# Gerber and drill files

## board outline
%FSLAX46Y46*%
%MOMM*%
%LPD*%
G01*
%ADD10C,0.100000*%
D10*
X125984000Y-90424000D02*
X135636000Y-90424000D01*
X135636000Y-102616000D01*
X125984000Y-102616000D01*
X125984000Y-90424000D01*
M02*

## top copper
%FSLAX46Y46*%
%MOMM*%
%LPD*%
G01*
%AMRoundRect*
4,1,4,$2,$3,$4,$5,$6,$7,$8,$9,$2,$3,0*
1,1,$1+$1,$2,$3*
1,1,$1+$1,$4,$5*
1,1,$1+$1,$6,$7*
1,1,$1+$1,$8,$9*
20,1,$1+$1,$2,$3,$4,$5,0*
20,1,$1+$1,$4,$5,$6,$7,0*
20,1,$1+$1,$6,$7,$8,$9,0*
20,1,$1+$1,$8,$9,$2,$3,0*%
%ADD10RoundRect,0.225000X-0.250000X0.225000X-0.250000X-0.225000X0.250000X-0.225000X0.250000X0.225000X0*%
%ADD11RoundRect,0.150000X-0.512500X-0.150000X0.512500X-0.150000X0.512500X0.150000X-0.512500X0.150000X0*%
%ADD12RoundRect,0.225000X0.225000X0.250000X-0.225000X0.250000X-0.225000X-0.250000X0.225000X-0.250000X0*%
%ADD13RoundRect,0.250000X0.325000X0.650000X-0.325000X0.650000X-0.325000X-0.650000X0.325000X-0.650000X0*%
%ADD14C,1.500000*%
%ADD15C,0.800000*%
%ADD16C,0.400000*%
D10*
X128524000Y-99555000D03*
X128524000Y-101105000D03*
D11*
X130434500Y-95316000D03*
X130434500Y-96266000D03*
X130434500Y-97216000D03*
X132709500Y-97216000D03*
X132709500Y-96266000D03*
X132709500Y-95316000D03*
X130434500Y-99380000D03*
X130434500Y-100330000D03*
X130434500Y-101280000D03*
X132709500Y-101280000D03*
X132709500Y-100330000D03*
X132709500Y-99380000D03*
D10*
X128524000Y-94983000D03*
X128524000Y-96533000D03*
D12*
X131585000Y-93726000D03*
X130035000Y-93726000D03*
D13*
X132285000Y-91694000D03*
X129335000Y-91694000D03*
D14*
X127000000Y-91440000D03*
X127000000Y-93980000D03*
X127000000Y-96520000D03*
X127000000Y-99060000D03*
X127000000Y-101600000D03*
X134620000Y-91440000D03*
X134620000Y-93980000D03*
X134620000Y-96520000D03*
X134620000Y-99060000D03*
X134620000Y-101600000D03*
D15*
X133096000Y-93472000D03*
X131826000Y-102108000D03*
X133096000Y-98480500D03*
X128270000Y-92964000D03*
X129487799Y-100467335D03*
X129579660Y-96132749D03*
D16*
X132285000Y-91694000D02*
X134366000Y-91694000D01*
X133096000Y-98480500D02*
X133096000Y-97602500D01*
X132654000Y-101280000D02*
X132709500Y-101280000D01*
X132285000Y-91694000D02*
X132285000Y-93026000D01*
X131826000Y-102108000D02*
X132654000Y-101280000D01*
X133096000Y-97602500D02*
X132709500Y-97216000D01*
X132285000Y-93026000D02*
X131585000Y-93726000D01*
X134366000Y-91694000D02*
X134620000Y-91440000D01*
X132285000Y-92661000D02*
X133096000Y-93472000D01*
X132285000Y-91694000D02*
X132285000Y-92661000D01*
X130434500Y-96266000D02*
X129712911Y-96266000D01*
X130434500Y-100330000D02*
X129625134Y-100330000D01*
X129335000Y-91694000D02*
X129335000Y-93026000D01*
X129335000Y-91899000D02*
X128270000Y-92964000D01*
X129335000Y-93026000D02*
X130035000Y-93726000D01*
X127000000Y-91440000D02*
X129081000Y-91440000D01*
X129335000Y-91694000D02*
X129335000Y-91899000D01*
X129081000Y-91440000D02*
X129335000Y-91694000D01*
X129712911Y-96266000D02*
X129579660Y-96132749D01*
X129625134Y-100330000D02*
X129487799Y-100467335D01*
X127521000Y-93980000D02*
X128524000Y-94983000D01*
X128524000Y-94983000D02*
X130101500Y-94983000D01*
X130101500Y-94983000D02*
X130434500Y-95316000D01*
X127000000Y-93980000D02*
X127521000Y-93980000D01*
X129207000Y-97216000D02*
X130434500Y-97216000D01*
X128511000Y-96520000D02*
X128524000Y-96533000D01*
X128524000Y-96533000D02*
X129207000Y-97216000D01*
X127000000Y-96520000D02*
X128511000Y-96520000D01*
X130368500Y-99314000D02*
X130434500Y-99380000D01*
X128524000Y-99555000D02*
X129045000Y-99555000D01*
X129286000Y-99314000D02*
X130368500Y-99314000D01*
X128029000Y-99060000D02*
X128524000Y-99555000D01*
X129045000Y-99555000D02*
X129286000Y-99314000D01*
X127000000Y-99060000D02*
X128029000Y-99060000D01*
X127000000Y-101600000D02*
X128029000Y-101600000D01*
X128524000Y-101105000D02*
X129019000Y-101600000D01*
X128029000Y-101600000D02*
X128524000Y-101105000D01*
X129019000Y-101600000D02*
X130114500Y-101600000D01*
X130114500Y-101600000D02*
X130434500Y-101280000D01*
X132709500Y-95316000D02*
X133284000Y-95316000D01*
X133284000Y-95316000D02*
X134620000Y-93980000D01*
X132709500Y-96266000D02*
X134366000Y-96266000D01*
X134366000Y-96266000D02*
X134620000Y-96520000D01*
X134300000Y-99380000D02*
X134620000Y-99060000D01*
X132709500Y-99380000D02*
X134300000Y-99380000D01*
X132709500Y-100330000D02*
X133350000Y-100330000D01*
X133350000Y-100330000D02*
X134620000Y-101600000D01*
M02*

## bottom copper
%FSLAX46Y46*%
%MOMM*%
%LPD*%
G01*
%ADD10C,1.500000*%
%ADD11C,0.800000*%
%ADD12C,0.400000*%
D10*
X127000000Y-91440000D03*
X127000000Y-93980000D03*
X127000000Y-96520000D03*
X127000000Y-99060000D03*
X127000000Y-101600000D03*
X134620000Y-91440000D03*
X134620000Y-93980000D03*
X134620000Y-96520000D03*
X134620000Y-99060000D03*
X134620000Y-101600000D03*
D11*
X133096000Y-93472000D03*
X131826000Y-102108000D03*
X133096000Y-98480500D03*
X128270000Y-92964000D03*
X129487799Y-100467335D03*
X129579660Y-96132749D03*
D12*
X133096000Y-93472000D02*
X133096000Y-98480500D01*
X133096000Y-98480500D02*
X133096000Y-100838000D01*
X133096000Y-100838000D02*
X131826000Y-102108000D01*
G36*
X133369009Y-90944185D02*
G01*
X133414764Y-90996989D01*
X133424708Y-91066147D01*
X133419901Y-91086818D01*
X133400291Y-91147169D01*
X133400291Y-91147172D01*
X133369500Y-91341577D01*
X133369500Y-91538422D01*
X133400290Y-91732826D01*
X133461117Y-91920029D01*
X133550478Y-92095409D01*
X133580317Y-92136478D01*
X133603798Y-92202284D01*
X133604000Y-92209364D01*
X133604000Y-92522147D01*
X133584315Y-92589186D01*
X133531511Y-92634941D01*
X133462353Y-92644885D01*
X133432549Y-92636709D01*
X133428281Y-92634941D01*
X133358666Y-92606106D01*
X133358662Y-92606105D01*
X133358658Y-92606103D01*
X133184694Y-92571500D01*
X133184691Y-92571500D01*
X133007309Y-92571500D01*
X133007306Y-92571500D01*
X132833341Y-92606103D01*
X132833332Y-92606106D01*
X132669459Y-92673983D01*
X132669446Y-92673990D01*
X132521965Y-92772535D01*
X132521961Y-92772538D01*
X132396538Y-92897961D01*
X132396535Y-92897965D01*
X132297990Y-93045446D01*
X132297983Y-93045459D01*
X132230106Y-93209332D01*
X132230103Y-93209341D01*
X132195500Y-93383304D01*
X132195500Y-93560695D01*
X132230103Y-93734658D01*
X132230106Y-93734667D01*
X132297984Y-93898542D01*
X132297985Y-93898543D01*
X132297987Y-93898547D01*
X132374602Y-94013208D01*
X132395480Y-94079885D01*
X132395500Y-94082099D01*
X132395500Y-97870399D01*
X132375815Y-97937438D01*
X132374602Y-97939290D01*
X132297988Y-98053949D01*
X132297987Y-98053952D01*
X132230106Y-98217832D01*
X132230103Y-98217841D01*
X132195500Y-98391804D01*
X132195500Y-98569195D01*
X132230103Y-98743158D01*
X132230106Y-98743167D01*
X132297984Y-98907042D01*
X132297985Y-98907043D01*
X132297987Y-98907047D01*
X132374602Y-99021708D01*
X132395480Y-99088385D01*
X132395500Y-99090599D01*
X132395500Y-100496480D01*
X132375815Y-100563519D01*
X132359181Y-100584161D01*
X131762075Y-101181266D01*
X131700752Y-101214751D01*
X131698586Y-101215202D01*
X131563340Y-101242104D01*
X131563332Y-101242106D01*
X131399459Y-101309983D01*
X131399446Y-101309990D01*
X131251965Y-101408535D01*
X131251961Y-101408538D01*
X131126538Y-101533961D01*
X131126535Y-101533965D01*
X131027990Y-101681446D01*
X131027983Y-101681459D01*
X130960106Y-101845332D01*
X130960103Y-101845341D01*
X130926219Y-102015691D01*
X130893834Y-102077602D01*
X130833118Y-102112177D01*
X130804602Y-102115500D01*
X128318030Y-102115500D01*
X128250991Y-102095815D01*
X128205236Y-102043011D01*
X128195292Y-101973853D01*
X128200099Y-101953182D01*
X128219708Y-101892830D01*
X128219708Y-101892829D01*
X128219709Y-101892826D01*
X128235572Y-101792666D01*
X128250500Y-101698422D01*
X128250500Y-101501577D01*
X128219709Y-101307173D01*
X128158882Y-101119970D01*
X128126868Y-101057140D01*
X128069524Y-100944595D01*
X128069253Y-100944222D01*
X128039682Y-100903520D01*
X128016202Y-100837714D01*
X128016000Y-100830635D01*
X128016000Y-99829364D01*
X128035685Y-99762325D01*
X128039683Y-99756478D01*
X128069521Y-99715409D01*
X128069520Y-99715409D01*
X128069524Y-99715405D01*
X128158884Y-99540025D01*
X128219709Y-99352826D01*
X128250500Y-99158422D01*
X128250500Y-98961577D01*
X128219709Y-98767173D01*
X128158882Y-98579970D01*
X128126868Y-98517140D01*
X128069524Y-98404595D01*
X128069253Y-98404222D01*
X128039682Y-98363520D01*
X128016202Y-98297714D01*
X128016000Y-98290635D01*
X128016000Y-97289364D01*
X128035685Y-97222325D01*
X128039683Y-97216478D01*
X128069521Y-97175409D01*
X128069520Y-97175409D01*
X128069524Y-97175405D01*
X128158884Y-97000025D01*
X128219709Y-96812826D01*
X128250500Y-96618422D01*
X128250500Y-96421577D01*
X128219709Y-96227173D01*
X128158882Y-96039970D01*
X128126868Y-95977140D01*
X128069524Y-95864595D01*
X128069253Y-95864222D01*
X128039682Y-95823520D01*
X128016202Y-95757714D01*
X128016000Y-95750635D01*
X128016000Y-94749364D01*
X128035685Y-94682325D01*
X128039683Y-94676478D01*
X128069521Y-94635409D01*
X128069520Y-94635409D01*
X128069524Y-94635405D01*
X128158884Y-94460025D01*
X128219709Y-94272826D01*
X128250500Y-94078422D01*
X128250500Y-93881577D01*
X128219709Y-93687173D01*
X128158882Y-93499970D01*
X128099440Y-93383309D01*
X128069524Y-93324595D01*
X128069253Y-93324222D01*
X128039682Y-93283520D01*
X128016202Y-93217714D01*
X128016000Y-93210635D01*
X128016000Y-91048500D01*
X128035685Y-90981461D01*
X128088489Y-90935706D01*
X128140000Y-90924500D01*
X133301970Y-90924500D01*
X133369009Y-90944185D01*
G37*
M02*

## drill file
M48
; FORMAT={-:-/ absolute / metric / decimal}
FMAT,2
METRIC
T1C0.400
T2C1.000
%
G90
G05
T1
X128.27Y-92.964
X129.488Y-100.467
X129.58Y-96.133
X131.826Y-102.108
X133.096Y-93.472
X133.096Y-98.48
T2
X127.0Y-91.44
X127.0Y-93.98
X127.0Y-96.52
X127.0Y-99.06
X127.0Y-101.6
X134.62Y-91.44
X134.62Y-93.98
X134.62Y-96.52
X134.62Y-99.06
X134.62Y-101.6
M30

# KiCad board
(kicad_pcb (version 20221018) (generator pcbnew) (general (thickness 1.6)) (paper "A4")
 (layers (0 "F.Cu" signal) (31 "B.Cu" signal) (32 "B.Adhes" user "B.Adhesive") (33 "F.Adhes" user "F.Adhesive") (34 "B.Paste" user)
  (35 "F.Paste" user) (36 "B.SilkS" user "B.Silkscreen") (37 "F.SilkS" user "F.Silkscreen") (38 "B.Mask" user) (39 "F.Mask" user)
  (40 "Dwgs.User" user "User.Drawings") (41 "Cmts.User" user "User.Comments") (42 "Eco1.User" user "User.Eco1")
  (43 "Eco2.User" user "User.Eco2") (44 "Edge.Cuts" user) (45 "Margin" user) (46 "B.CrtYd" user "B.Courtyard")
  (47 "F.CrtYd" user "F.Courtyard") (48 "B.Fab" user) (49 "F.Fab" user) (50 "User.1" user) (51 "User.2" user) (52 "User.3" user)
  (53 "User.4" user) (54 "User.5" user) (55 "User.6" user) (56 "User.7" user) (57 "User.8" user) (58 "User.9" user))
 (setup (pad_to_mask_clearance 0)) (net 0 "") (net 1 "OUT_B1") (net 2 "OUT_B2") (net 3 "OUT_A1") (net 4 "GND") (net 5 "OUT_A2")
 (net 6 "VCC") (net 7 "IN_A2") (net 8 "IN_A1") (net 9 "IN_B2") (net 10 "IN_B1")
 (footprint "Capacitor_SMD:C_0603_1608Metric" (layer "F.Cu") (at 128.524 100.33 -90)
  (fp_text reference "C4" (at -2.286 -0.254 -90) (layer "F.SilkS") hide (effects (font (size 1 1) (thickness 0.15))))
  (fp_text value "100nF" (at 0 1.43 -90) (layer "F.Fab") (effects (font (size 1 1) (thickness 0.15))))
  (pad "1" smd roundrect (at -0.775 0 270) (size 0.9 0.95) (layers "F.Cu" "F.Paste" "F.Mask") (roundrect_rratio 0.25) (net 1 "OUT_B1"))
  (pad "2" smd roundrect (at 0.775 0 270) (size 0.9 0.95) (layers "F.Cu" "F.Paste" "F.Mask") (roundrect_rratio 0.25) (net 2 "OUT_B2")))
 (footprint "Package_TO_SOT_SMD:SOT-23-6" (layer "F.Cu") (at 131.572 96.266)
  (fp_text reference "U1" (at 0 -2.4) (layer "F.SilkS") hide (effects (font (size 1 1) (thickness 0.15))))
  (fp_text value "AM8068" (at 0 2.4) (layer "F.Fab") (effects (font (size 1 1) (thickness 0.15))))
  (pad "1" smd roundrect (at -1.1375 -0.95) (size 1.325 0.6) (layers "F.Cu" "F.Paste" "F.Mask") (roundrect_rratio 0.25) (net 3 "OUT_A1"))
  (pad "2" smd roundrect (at -1.1375 0) (size 1.325 0.6) (layers "F.Cu" "F.Paste" "F.Mask") (roundrect_rratio 0.25) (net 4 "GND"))
  (pad "3" smd roundrect (at -1.1375 0.95) (size 1.325 0.6) (layers "F.Cu" "F.Paste" "F.Mask") (roundrect_rratio 0.25) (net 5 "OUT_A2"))
  (pad "4" smd roundrect (at 1.1375 0.95) (size 1.325 0.6) (layers "F.Cu" "F.Paste" "F.Mask") (roundrect_rratio 0.25) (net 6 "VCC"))
  (pad "5" smd roundrect (at 1.1375 0) (size 1.325 0.6) (layers "F.Cu" "F.Paste" "F.Mask") (roundrect_rratio 0.25) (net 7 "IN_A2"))
  (pad "6" smd roundrect (at 1.1375 -0.95) (size 1.325 0.6) (layers "F.Cu" "F.Paste" "F.Mask") (roundrect_rratio 0.25) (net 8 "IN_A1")))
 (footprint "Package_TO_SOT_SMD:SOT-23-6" (layer "F.Cu") (at 131.572 100.33)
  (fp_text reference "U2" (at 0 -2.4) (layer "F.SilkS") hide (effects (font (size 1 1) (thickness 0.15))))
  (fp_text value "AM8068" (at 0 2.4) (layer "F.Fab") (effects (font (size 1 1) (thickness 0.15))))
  (pad "1" smd roundrect (at -1.1375 -0.95) (size 1.325 0.6) (layers "F.Cu" "F.Paste" "F.Mask") (roundrect_rratio 0.25) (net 1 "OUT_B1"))
  (pad "2" smd roundrect (at -1.1375 0) (size 1.325 0.6) (layers "F.Cu" "F.Paste" "F.Mask") (roundrect_rratio 0.25) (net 4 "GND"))
  (pad "3" smd roundrect (at -1.1375 0.95) (size 1.325 0.6) (layers "F.Cu" "F.Paste" "F.Mask") (roundrect_rratio 0.25) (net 2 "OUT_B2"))
  (pad "4" smd roundrect (at 1.1375 0.95) (size 1.325 0.6) (layers "F.Cu" "F.Paste" "F.Mask") (roundrect_rratio 0.25) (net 6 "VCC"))
  (pad "5" smd roundrect (at 1.1375 0) (size 1.325 0.6) (layers "F.Cu" "F.Paste" "F.Mask") (roundrect_rratio 0.25) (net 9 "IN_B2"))
  (pad "6" smd roundrect (at 1.1375 -0.95) (size 1.325 0.6) (layers "F.Cu" "F.Paste" "F.Mask") (roundrect_rratio 0.25) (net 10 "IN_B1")))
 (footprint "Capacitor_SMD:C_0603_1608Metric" (layer "F.Cu") (at 128.524 95.758 -90)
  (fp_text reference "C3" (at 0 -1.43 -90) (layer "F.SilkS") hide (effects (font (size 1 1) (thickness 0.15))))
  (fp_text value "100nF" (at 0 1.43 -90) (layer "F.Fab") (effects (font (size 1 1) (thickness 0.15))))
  (pad "1" smd roundrect (at -0.775 0 270) (size 0.9 0.95) (layers "F.Cu" "F.Paste" "F.Mask") (roundrect_rratio 0.25) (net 3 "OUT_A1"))
  (pad "2" smd roundrect (at 0.775 0 270) (size 0.9 0.95) (layers "F.Cu" "F.Paste" "F.Mask") (roundrect_rratio 0.25) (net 5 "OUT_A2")))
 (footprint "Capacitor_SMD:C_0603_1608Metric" (layer "F.Cu") (at 130.81 93.726 180)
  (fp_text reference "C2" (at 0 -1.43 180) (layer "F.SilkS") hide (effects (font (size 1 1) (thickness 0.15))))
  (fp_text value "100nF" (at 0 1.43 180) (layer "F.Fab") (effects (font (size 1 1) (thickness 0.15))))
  (pad "1" smd roundrect (at -0.775 0 180) (size 0.9 0.95) (layers "F.Cu" "F.Paste" "F.Mask") (roundrect_rratio 0.25) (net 6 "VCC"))
  (pad "2" smd roundrect (at 0.775 0 180) (size 0.9 0.95) (layers "F.Cu" "F.Paste" "F.Mask") (roundrect_rratio 0.25) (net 4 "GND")))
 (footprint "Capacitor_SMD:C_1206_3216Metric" (layer "F.Cu") (at 130.81 91.694 180)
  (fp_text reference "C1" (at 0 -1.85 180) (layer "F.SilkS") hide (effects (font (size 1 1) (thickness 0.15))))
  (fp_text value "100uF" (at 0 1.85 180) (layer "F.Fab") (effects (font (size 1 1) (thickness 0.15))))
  (pad "1" smd roundrect (at -1.475 0 180) (size 1.15 1.8) (layers "F.Cu" "F.Paste" "F.Mask") (roundrect_rratio 0.2173913043) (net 6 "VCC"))
  (pad "2" smd roundrect (at 1.475 0 180) (size 1.15 1.8) (layers "F.Cu" "F.Paste" "F.Mask") (roundrect_rratio 0.2173913043) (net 4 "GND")))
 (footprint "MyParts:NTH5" (layer "F.Cu") (at 127 96.52)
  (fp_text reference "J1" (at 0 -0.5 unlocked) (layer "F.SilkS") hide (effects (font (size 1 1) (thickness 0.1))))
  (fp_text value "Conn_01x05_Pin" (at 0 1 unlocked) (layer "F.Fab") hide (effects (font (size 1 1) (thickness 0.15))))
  (pad "1" thru_hole circle (at 0 -5.08) (size 1.5 1.5) (drill 1) (layers "*.Cu" "*.Mask") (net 4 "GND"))
  (pad "2" thru_hole circle (at 0 -2.54) (size 1.5 1.5) (drill 1) (layers "*.Cu" "*.Mask") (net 3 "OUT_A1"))
  (pad "3" thru_hole circle (at 0 0) (size 1.5 1.5) (drill 1) (layers "*.Cu" "*.Mask") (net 5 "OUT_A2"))
  (pad "4" thru_hole circle (at 0 2.54) (size 1.5 1.5) (drill 1) (layers "*.Cu" "*.Mask") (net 1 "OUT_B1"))
  (pad "5" thru_hole circle (at 0 5.08) (size 1.5 1.5) (drill 1) (layers "*.Cu" "*.Mask") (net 2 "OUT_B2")))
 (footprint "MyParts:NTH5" (layer "F.Cu") (at 134.62 96.52)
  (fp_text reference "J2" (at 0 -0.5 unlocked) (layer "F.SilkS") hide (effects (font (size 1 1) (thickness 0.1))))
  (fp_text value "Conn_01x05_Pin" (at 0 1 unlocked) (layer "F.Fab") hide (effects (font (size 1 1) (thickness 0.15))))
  (pad "1" thru_hole circle (at 0 -5.08) (size 1.5 1.5) (drill 1) (layers "*.Cu" "*.Mask") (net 6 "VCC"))
  (pad "2" thru_hole circle (at 0 -2.54) (size 1.5 1.5) (drill 1) (layers "*.Cu" "*.Mask") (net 8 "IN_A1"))
  (pad "3" thru_hole circle (at 0 0) (size 1.5 1.5) (drill 1) (layers "*.Cu" "*.Mask") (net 7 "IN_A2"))
  (pad "4" thru_hole circle (at 0 2.54) (size 1.5 1.5) (drill 1) (layers "*.Cu" "*.Mask") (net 10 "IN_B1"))
  (pad "5" thru_hole circle (at 0 5.08) (size 1.5 1.5) (drill 1) (layers "*.Cu" "*.Mask") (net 9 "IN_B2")))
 (gr_rect (start 125.984 90.424) (end 135.636 102.616) (stroke (width 0.1) (type default)) (fill none) (layer "Edge.Cuts"))
 (segment (start 132.285 91.694) (end 134.366 91.694) (width 0.4) (layer "F.Cu") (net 6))
 (segment (start 133.096 98.4805) (end 133.096 97.6025) (width 0.4) (layer "F.Cu") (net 6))
 (segment (start 132.654 101.28) (end 132.7095 101.28) (width 0.4) (layer "F.Cu") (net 6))
 (segment (start 132.285 91.694) (end 132.285 93.026) (width 0.4) (layer "F.Cu") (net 6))
 (segment (start 131.826 102.108) (end 132.654 101.28) (width 0.4) (layer "F.Cu") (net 6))
 (segment (start 133.096 97.6025) (end 132.7095 97.216) (width 0.4) (layer "F.Cu") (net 6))
 (segment (start 132.285 93.026) (end 131.585 93.726) (width 0.4) (layer "F.Cu") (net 6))
 (segment (start 134.366 91.694) (end 134.62 91.44) (width 0.4) (layer "F.Cu") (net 6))
 (segment (start 132.285 92.661) (end 133.096 93.472) (width 0.4) (layer "F.Cu") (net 6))
 (segment (start 132.285 91.694) (end 132.285 92.661) (width 0.4) (layer "F.Cu") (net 6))
 (via (at 133.096 93.472) (size 0.8) (drill 0.4) (layers "F.Cu" "B.Cu") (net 6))
 (via (at 131.826 102.108) (size 0.8) (drill 0.4) (layers "F.Cu" "B.Cu") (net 6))
 (via (at 133.096 98.4805) (size 0.8) (drill 0.4) (layers "F.Cu" "B.Cu") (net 6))
 (segment (start 133.096 93.472) (end 133.096 98.4805) (width 0.4) (layer "B.Cu") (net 6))
 (segment (start 133.096 98.4805) (end 133.096 100.838) (width 0.4) (layer "B.Cu") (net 6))
 (segment (start 133.096 100.838) (end 131.826 102.108) (width 0.4) (layer "B.Cu") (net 6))
 (segment (start 130.4345 96.266) (end 129.712911 96.266) (width 0.4) (layer "F.Cu") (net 4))
 (segment (start 130.4345 100.33) (end 129.625134 100.33) (width 0.4) (layer "F.Cu") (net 4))
 (segment (start 129.335 91.694) (end 129.335 93.026) (width 0.4) (layer "F.Cu") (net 4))
 (segment (start 129.335 91.899) (end 128.27 92.964) (width 0.4) (layer "F.Cu") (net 4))
 (segment (start 129.335 93.026) (end 130.035 93.726) (width 0.4) (layer "F.Cu") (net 4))
 (segment (start 127 91.44) (end 129.081 91.44) (width 0.4) (layer "F.Cu") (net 4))
 (segment (start 129.335 91.694) (end 129.335 91.899) (width 0.4) (layer "F.Cu") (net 4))
 (segment (start 129.081 91.44) (end 129.335 91.694) (width 0.4) (layer "F.Cu") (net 4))
 (segment (start 129.712911 96.266) (end 129.57966 96.132749) (width 0.4) (layer "F.Cu") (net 4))
 (segment (start 129.625134 100.33) (end 129.487799 100.467335) (width 0.4) (layer "F.Cu") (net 4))
 (via (at 128.27 92.964) (size 0.8) (drill 0.4) (layers "F.Cu" "B.Cu") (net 4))
 (via (at 129.487799 100.467335) (size 0.8) (drill 0.4) (layers "F.Cu" "B.Cu") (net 4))
 (via (at 129.57966 96.132749) (size 0.8) (drill 0.4) (layers "F.Cu" "B.Cu") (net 4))
 (segment (start 127.521 93.98) (end 128.524 94.983) (width 0.4) (layer "F.Cu") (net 3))
 (segment (start 128.524 94.983) (end 130.1015 94.983) (width 0.4) (layer "F.Cu") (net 3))
 (segment (start 130.1015 94.983) (end 130.4345 95.316) (width 0.4) (layer "F.Cu") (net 3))
 (segment (start 127 93.98) (end 127.521 93.98) (width 0.4) (layer "F.Cu") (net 3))
 (segment (start 129.207 97.216) (end 130.4345 97.216) (width 0.4) (layer "F.Cu") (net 5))
 (segment (start 128.511 96.52) (end 128.524 96.533) (width 0.4) (layer "F.Cu") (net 5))
 (segment (start 128.524 96.533) (end 129.207 97.216) (width 0.4) (layer "F.Cu") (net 5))
 (segment (start 127 96.52) (end 128.511 96.52) (width 0.4) (layer "F.Cu") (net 5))
 (segment (start 130.3685 99.314) (end 130.4345 99.38) (width 0.4) (layer "F.Cu") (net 1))
 (segment (start 128.524 99.555) (end 129.045 99.555) (width 0.4) (layer "F.Cu") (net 1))
 (segment (start 129.286 99.314) (end 130.3685 99.314) (width 0.4) (layer "F.Cu") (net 1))
 (segment (start 128.029 99.06) (end 128.524 99.555) (width 0.4) (layer "F.Cu") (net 1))
 (segment (start 129.045 99.555) (end 129.286 99.314) (width 0.4) (layer "F.Cu") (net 1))
 (segment (start 127 99.06) (end 128.029 99.06) (width 0.4) (layer "F.Cu") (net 1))
 (segment (start 127 101.6) (end 128.029 101.6) (width 0.4) (layer "F.Cu") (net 2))
 (segment (start 128.524 101.105) (end 129.019 101.6) (width 0.4) (layer "F.Cu") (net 2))
 (segment (start 128.029 101.6) (end 128.524 101.105) (width 0.4) (layer "F.Cu") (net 2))
 (segment (start 129.019 101.6) (end 130.1145 101.6) (width 0.4) (layer "F.Cu") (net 2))
 (segment (start 130.1145 101.6) (end 130.4345 101.28) (width 0.4) (layer "F.Cu") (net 2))
 (segment (start 132.7095 95.316) (end 133.284 95.316) (width 0.4) (layer "F.Cu") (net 8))
 (segment (start 133.284 95.316) (end 134.62 93.98) (width 0.4) (layer "F.Cu") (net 8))
 (segment (start 132.7095 96.266) (end 134.366 96.266) (width 0.4) (layer "F.Cu") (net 7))
 (segment (start 134.366 96.266) (end 134.62 96.52) (width 0.4) (layer "F.Cu") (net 7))
 (segment (start 134.3 99.38) (end 134.62 99.06) (width 0.4) (layer "F.Cu") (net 10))
 (segment (start 132.7095 99.38) (end 134.3 99.38) (width 0.4) (layer "F.Cu") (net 10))
 (segment (start 132.7095 100.33) (end 133.35 100.33) (width 0.4) (layer "F.Cu") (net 9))
 (segment (start 133.35 100.33) (end 134.62 101.6) (width 0.4) (layer "F.Cu") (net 9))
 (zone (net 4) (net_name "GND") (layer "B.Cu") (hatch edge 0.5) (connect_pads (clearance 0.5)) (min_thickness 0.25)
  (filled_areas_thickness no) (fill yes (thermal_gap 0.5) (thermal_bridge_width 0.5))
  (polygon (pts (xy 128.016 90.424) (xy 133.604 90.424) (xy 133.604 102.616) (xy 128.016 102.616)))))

